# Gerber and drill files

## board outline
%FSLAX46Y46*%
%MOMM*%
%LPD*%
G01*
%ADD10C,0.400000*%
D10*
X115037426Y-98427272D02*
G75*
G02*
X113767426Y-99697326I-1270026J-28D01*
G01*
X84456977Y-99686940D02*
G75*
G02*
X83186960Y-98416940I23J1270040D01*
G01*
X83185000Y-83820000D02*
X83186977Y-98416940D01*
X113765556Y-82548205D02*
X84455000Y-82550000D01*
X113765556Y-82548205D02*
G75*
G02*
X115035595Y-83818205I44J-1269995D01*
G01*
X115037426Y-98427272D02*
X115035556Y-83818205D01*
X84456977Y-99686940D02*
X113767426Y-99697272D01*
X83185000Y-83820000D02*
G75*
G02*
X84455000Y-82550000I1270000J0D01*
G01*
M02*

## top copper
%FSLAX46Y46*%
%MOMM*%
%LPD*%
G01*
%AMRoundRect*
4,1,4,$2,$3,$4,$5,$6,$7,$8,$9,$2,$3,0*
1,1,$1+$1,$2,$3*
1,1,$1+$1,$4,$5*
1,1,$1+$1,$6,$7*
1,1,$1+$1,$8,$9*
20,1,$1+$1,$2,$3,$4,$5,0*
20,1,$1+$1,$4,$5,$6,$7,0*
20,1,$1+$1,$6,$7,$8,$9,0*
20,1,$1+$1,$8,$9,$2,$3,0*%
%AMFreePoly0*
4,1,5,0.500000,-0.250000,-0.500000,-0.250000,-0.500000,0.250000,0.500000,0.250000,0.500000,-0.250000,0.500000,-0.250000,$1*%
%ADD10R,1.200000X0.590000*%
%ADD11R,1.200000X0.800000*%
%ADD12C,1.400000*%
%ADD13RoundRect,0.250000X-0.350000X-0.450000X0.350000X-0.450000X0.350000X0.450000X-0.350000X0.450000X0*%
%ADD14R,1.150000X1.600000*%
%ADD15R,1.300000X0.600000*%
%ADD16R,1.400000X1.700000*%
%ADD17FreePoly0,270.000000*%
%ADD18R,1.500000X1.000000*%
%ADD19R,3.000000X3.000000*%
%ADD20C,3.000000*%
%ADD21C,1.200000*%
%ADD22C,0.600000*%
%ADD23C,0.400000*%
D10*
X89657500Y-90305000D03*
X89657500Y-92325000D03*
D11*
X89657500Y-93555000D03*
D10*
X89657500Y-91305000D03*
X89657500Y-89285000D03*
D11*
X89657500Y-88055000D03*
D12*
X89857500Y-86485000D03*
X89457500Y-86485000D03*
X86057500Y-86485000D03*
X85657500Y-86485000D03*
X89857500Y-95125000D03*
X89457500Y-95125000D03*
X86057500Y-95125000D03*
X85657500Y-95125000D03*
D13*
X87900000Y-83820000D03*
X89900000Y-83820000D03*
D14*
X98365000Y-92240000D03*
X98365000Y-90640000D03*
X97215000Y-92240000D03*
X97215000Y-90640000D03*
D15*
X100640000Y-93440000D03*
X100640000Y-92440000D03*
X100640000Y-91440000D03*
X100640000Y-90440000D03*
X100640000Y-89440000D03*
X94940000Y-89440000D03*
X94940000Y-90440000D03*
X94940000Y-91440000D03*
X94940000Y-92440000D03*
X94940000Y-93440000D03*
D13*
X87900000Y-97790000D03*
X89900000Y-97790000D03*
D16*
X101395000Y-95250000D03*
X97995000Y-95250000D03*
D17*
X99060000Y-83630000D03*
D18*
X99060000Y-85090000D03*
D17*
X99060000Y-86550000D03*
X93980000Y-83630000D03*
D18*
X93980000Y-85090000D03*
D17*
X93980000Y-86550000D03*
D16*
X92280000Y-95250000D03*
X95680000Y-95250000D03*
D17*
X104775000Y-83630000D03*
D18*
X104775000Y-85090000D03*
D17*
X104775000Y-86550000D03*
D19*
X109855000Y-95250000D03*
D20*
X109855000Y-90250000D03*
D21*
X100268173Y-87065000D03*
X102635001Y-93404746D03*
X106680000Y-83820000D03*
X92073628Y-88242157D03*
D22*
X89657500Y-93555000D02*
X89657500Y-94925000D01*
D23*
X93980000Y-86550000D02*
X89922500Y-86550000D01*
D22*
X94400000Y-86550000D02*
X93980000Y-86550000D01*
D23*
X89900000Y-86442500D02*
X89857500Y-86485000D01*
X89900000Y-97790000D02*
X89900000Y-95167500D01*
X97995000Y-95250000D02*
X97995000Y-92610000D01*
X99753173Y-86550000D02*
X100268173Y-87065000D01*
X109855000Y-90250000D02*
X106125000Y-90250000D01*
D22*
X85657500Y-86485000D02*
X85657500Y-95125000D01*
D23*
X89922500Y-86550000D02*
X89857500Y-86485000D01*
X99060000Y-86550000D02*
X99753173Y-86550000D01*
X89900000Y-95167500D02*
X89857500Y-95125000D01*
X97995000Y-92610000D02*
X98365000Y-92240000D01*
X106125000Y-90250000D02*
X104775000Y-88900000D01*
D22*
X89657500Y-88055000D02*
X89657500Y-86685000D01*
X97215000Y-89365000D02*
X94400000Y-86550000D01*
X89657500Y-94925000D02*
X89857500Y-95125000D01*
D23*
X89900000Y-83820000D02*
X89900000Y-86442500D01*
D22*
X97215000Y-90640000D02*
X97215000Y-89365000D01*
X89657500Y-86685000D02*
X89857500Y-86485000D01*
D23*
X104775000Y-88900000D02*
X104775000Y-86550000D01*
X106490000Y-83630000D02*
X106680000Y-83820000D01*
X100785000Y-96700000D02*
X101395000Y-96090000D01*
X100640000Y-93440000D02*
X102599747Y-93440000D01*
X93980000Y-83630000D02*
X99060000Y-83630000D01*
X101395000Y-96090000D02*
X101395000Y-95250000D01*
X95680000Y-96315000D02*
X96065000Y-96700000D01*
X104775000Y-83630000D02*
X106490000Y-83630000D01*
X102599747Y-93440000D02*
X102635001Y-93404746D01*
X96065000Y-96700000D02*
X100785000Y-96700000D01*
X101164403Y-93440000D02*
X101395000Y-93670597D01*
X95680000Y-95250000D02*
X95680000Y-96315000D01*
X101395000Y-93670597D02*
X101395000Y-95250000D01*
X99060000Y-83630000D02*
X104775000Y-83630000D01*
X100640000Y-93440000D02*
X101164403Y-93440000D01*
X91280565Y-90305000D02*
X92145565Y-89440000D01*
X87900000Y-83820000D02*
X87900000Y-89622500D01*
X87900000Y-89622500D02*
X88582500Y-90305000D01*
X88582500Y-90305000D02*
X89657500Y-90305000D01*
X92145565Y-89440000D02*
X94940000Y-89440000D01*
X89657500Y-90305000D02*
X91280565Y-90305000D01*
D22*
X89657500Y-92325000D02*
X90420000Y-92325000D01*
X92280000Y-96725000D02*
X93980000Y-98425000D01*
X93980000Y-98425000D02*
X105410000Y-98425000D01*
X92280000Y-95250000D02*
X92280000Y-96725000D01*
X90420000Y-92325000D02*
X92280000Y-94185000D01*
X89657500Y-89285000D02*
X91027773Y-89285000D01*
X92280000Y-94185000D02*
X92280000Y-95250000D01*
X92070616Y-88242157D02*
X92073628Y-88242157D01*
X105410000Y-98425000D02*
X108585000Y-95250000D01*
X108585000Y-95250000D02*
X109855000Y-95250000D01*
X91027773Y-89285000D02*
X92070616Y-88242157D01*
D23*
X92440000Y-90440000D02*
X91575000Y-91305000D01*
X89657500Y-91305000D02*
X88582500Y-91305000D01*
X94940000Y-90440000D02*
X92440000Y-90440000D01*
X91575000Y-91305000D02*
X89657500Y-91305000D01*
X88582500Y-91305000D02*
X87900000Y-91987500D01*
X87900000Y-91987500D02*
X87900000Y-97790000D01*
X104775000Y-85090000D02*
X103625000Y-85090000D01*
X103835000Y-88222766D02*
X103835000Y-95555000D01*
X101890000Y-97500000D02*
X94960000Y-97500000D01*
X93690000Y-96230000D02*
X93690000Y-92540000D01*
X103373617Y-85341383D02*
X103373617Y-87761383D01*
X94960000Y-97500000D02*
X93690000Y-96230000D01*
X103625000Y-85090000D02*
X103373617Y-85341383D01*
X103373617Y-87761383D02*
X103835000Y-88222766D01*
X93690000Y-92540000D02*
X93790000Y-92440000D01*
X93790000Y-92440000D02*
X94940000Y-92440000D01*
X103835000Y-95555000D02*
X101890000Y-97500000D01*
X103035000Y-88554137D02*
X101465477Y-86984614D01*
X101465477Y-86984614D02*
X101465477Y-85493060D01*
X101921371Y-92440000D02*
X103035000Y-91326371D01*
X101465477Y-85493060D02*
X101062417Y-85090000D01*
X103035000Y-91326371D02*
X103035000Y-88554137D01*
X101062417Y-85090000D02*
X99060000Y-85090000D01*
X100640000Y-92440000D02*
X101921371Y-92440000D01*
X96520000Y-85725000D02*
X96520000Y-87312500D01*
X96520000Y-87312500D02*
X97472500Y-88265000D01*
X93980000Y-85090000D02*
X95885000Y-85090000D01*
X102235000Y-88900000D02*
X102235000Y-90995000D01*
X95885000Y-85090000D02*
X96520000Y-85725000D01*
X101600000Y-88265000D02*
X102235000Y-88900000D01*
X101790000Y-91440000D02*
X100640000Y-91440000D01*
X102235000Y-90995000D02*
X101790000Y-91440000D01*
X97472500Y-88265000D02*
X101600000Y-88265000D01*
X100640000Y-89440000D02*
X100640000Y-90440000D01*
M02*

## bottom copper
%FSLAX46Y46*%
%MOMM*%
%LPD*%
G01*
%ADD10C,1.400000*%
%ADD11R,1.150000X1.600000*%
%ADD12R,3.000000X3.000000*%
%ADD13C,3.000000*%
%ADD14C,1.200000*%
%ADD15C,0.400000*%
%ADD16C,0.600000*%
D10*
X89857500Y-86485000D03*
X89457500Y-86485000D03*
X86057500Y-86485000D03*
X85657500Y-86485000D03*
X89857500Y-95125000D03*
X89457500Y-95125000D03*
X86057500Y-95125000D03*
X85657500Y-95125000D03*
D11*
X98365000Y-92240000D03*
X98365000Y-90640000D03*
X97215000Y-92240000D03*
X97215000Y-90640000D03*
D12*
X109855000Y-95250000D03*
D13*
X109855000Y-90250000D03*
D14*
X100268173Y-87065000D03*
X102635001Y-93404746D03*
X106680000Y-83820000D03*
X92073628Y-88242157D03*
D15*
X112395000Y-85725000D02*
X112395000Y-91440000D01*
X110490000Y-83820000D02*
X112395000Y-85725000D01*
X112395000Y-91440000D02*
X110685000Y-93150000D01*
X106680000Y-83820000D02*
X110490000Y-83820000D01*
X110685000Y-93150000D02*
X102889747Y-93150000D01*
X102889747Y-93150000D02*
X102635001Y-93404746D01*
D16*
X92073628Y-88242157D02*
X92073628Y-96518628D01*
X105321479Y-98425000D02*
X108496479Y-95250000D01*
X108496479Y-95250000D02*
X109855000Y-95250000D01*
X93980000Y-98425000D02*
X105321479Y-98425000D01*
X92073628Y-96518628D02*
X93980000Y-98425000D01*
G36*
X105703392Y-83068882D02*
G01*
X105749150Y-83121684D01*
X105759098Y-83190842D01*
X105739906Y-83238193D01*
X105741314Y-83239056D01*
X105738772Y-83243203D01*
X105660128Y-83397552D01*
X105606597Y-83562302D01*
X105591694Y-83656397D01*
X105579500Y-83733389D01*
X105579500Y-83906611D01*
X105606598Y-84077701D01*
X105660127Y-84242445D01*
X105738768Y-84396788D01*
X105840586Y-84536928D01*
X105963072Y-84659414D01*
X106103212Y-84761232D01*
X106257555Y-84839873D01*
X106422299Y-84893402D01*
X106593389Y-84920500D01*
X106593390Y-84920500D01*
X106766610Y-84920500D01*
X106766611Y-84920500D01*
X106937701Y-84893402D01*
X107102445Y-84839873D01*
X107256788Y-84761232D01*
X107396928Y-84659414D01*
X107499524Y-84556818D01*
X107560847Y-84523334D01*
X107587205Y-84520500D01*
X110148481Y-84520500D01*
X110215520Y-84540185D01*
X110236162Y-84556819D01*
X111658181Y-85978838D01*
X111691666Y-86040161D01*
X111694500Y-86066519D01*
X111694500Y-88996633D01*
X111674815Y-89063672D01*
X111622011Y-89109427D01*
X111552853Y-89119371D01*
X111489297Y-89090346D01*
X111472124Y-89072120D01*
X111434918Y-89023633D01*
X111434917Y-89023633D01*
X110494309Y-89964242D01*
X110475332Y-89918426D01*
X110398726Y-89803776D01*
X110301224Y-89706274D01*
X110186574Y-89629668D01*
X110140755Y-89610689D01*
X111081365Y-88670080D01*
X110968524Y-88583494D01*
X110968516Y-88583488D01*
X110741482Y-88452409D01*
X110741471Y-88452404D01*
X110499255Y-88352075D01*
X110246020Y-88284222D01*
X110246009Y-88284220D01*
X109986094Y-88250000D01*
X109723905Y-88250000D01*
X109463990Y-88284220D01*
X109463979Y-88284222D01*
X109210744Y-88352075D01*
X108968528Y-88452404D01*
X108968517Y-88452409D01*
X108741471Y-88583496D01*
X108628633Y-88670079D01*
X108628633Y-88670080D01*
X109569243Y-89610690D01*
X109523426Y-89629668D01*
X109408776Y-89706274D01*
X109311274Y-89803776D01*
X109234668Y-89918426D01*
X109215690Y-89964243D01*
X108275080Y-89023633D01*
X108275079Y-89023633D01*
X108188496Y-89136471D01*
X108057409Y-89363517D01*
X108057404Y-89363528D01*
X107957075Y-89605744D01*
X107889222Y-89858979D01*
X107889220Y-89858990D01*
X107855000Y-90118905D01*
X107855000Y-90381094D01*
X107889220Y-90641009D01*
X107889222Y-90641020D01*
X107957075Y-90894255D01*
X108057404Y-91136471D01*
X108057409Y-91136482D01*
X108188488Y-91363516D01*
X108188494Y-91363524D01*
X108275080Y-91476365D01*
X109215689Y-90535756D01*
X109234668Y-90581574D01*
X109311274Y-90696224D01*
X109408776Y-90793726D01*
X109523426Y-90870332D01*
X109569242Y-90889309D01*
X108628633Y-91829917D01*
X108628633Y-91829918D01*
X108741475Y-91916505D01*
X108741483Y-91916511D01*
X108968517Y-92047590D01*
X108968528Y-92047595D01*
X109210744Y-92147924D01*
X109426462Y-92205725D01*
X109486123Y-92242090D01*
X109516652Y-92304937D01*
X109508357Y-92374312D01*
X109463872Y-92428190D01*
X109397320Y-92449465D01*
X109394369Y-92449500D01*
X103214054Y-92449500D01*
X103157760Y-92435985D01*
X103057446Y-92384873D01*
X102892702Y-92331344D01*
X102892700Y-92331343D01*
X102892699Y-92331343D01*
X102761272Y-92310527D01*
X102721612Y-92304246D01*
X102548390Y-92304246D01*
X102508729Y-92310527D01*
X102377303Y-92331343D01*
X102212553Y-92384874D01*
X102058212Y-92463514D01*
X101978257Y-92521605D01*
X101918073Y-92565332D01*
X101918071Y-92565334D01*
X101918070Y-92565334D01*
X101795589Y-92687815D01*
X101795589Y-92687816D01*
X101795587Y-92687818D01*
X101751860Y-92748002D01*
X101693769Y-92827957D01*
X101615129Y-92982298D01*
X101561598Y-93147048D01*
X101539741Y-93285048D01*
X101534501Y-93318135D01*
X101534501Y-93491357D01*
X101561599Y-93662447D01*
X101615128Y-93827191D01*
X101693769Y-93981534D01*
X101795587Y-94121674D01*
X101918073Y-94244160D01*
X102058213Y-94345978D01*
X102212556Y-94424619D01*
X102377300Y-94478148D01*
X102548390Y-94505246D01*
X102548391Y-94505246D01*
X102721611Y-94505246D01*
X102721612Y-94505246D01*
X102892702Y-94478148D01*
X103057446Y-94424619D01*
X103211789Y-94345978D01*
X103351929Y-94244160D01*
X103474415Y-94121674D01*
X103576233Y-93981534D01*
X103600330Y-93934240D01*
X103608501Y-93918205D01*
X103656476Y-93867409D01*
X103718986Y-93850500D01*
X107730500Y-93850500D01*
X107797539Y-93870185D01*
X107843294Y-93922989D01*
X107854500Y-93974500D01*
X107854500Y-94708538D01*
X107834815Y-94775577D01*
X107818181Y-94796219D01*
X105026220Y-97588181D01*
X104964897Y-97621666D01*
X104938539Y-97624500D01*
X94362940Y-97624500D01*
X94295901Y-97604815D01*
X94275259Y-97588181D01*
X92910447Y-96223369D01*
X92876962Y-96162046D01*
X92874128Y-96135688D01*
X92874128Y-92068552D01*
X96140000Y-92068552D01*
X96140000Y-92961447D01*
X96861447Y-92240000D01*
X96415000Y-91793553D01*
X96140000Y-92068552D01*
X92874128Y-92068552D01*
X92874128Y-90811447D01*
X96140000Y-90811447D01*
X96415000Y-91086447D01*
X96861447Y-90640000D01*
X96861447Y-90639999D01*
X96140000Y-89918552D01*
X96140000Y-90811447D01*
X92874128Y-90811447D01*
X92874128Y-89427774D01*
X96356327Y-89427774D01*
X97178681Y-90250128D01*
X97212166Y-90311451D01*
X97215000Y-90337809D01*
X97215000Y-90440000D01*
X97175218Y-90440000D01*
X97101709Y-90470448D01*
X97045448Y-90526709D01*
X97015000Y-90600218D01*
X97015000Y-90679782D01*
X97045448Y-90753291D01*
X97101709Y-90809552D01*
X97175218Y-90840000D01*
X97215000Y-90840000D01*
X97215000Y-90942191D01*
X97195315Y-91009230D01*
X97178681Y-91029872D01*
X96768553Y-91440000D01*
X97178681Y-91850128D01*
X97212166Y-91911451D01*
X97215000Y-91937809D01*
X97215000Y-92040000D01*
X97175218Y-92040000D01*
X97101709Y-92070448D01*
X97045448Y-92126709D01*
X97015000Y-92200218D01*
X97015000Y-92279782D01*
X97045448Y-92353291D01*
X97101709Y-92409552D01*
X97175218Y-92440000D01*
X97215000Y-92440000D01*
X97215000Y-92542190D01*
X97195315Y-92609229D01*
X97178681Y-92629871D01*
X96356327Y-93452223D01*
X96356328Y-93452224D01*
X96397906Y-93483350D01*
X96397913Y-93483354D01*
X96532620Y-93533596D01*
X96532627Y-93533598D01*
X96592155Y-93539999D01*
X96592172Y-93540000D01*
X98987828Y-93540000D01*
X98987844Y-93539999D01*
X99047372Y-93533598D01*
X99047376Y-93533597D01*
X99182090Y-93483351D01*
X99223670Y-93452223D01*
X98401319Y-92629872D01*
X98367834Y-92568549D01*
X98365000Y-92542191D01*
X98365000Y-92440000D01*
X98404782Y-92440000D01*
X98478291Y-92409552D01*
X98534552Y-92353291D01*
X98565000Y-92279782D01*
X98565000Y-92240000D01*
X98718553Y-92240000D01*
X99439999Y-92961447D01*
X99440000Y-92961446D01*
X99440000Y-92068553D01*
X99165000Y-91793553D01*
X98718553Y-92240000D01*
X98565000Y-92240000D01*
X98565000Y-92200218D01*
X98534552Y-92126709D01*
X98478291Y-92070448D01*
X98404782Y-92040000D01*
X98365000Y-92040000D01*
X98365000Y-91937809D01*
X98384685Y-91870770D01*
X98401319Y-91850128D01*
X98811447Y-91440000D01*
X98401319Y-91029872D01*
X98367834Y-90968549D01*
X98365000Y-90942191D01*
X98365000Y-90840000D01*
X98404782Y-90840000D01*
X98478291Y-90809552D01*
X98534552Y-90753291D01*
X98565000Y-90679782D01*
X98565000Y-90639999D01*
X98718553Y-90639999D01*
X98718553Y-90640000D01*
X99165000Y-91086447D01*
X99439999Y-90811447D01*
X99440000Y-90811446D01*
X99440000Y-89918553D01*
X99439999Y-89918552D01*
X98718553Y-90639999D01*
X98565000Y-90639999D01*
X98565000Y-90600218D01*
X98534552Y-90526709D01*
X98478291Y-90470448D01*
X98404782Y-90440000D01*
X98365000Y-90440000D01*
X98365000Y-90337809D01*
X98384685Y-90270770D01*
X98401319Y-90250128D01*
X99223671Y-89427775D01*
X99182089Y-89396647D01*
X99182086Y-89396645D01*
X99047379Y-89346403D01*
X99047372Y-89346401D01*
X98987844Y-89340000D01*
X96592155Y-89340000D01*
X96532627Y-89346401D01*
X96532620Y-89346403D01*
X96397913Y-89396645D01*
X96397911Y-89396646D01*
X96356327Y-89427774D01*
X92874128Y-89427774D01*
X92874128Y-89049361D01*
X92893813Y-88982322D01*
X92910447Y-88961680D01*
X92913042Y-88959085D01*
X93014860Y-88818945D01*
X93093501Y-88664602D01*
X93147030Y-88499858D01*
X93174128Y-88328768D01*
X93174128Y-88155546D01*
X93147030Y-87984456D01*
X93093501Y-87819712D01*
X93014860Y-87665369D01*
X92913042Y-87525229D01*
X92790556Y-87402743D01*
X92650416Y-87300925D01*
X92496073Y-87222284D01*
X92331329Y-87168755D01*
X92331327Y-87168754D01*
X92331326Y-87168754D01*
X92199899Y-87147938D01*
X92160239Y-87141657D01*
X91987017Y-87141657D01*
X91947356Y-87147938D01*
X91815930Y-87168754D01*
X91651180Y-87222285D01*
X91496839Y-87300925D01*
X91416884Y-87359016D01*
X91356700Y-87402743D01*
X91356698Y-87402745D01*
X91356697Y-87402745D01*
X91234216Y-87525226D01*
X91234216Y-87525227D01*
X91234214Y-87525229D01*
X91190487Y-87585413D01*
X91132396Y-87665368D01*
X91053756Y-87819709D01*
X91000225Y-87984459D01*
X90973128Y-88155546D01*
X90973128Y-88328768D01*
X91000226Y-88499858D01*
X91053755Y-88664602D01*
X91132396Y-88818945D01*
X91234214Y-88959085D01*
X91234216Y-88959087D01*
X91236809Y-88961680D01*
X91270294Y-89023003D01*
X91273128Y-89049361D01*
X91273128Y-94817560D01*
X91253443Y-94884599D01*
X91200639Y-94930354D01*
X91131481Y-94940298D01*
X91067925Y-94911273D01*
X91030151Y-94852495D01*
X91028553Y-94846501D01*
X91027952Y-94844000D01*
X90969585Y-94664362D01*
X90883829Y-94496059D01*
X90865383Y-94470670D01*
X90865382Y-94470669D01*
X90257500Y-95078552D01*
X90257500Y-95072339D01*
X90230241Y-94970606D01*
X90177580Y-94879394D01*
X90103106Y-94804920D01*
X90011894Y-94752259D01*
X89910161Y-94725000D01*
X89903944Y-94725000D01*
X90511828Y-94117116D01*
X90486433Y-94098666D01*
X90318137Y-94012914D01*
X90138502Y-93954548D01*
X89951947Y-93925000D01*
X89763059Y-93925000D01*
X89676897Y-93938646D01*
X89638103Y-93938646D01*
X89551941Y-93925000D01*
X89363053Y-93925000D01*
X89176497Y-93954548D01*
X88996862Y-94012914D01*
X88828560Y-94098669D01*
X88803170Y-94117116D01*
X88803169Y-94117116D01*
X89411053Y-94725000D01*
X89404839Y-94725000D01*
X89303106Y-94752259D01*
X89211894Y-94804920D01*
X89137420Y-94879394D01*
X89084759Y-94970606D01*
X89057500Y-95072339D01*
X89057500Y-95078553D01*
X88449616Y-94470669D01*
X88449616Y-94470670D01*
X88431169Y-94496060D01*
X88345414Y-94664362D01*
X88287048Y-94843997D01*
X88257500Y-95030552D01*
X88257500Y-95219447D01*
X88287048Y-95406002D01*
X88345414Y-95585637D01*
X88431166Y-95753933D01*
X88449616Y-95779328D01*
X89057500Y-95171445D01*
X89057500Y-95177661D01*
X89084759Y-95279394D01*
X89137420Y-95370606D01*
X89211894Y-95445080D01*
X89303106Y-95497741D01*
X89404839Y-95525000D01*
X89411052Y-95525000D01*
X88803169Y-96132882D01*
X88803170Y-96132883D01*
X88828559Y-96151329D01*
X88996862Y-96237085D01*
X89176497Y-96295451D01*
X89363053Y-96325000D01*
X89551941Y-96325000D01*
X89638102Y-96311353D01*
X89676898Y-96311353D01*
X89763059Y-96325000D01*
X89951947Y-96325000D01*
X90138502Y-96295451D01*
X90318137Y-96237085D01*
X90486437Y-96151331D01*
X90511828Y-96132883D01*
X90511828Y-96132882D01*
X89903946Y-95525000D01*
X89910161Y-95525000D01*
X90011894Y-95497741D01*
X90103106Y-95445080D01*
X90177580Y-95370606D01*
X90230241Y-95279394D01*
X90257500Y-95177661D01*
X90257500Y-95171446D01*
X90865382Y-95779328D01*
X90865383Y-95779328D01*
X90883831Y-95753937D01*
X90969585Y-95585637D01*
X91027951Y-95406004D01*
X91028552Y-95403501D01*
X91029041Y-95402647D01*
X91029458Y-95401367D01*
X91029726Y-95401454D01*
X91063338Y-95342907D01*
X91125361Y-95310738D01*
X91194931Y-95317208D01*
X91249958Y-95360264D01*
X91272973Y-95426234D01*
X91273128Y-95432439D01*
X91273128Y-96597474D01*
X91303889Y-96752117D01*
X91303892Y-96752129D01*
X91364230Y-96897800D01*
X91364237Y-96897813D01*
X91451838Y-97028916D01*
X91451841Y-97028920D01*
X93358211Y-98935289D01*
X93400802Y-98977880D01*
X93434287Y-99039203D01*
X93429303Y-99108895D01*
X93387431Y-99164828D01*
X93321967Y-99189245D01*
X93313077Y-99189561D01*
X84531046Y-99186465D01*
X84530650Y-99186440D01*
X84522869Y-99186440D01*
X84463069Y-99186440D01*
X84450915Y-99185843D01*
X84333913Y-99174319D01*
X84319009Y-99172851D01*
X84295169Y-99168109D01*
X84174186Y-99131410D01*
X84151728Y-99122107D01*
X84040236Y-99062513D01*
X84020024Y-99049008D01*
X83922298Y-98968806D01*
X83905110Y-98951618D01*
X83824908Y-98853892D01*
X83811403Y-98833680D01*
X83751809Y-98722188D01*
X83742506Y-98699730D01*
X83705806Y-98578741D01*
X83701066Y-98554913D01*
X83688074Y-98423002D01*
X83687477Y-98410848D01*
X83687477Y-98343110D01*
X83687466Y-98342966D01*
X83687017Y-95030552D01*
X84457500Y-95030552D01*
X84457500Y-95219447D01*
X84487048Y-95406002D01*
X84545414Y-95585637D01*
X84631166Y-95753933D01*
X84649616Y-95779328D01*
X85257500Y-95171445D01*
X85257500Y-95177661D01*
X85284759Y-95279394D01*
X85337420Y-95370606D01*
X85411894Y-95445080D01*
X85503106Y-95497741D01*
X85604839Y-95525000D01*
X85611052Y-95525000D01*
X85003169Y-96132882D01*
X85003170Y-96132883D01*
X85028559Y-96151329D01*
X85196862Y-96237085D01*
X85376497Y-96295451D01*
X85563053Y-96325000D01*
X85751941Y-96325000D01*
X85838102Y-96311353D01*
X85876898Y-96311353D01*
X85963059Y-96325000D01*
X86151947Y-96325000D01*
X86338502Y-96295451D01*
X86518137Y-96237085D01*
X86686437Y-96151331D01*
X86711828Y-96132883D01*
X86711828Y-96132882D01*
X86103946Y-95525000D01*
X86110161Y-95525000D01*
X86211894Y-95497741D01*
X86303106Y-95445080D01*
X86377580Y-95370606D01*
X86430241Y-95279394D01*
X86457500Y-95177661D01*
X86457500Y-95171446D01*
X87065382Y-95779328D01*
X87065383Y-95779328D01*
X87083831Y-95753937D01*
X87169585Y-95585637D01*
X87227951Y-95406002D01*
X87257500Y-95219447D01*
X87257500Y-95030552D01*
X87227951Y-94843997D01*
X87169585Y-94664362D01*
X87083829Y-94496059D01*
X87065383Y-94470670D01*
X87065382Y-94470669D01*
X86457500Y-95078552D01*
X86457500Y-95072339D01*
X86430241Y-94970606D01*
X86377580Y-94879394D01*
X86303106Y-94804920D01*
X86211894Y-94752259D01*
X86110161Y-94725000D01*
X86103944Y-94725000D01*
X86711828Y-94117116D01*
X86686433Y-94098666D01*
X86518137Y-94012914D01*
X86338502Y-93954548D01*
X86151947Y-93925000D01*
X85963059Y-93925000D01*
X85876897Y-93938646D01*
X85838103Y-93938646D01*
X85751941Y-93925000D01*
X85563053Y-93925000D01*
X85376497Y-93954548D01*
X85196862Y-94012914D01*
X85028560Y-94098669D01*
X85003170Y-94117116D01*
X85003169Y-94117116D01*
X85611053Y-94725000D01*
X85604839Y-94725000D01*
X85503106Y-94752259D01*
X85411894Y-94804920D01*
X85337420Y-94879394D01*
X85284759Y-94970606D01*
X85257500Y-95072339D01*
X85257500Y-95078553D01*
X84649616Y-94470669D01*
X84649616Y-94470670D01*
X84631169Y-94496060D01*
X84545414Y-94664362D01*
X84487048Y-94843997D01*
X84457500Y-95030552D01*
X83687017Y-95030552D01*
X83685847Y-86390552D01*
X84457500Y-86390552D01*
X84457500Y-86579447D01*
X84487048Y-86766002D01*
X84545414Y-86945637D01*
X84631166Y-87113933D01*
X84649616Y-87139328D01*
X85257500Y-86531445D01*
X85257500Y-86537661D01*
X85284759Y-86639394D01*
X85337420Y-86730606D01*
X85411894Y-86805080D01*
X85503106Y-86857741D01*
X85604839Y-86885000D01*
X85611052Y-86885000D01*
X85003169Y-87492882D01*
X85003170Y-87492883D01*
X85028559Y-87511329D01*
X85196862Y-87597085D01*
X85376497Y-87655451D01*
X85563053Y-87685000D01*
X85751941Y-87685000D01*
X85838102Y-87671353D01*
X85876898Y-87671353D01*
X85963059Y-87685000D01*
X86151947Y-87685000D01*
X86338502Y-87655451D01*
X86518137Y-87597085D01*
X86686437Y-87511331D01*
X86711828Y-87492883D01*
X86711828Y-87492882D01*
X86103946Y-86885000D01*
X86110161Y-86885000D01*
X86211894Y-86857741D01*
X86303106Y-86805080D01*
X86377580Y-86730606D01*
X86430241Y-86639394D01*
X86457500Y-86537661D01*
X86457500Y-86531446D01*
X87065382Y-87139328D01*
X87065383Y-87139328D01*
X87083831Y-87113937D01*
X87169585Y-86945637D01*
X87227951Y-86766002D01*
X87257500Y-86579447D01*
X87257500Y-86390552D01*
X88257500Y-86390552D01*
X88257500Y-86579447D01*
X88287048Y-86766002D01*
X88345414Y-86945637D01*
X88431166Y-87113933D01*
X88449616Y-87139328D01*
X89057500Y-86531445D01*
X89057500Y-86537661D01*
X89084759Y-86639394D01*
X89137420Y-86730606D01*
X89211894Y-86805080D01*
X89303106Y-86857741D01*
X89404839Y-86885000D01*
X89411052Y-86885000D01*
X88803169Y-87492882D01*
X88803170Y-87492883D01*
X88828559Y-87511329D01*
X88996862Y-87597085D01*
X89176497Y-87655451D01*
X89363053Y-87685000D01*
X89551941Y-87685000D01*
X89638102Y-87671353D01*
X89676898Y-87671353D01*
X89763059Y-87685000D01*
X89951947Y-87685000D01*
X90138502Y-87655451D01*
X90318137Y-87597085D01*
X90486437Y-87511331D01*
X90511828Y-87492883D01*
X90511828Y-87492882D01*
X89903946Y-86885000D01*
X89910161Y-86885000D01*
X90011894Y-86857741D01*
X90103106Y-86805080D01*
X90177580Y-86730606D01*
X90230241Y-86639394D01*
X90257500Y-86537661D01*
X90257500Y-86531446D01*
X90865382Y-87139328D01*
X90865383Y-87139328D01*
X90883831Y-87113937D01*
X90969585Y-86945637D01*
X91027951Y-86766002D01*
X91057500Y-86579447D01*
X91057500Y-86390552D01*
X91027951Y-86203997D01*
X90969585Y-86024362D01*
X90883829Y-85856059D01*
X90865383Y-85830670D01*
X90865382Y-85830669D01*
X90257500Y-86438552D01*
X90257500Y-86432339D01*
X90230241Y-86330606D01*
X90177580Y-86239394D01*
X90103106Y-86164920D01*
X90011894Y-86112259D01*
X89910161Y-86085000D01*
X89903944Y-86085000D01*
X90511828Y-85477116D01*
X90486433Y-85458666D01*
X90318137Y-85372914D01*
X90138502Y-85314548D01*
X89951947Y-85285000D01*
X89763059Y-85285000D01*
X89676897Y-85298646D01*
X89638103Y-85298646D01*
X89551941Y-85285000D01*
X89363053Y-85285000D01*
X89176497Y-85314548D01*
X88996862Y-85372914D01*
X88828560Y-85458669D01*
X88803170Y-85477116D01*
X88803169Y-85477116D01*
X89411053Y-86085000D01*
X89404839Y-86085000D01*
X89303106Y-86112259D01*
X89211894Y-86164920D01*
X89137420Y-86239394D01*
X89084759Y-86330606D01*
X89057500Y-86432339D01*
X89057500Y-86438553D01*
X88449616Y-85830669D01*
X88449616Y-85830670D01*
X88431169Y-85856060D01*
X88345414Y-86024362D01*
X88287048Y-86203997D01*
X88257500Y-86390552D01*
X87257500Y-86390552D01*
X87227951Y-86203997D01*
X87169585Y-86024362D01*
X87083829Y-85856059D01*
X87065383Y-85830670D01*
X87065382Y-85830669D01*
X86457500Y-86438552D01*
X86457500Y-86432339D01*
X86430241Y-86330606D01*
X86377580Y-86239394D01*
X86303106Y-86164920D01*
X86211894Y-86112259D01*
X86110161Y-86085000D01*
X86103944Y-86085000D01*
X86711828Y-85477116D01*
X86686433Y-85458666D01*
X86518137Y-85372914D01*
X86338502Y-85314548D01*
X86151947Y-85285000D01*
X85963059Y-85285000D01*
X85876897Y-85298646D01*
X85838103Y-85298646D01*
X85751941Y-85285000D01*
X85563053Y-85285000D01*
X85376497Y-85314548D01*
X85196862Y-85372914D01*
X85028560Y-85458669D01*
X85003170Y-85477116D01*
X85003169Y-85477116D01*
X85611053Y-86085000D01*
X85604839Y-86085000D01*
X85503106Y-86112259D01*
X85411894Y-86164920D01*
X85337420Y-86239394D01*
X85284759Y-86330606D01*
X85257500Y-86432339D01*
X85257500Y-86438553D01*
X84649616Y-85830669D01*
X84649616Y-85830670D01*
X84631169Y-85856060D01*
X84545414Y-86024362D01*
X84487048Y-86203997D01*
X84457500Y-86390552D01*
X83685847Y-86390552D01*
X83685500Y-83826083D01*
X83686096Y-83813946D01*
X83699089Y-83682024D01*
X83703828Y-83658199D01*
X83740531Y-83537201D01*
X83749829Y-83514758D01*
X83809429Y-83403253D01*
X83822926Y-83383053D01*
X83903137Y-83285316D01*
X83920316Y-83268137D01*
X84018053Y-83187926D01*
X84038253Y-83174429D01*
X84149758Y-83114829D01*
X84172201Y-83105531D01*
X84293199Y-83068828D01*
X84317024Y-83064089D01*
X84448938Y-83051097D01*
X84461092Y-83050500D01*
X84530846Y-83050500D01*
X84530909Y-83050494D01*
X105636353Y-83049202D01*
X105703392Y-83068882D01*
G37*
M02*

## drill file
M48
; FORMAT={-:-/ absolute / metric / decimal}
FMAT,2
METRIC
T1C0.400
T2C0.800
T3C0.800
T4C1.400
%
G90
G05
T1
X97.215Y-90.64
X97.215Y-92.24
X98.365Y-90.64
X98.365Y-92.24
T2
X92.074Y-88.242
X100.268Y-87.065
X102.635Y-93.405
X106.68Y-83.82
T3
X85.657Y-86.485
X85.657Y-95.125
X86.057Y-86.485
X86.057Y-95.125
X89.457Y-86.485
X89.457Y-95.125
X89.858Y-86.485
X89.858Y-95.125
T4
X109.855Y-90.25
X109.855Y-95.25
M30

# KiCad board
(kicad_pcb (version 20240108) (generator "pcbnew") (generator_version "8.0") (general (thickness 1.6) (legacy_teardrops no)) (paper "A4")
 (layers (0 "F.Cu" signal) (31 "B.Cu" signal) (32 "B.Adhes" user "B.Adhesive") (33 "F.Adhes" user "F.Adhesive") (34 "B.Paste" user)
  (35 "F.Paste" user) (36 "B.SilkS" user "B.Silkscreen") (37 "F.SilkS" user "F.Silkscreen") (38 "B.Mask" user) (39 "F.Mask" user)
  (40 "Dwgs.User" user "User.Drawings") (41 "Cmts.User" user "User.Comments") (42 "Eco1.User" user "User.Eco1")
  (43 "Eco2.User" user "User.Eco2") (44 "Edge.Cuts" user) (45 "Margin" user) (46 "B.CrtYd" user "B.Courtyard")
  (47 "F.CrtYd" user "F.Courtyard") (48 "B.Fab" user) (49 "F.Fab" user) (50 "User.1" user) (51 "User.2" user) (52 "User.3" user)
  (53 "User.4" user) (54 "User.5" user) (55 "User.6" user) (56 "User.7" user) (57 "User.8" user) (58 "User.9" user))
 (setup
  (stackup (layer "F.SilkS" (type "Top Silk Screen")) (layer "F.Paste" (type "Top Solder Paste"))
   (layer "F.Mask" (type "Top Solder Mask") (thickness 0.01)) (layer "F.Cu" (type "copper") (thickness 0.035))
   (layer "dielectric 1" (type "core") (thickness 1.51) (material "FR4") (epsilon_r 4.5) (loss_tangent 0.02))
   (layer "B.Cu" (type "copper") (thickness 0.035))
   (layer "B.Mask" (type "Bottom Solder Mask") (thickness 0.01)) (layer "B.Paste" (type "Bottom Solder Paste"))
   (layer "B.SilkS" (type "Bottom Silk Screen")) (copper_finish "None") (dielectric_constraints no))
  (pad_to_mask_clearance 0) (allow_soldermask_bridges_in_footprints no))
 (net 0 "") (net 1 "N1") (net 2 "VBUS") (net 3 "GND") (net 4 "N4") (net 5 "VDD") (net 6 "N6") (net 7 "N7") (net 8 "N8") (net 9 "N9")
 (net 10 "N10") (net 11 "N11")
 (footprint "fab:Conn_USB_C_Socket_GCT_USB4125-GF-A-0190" (layer "F.Cu") (at 89.6575 90.805 -90)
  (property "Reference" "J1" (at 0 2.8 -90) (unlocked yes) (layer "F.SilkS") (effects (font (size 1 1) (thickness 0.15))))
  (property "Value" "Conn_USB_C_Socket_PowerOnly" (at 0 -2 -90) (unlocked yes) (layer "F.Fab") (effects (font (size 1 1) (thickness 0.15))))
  (pad "A5" smd rect (at -0.5 0 270) (size 0.59 1.2) (layers "F.Cu" "F.Paste" "F.Mask") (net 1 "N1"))
  (pad "A9" smd rect (at 1.52 0 270) (size 0.59 1.2) (layers "F.Cu" "F.Paste" "F.Mask") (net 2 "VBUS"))
  (pad "A12" smd rect (at 2.75 0 270) (size 0.8 1.2) (layers "F.Cu" "F.Paste" "F.Mask") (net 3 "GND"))
  (pad "B5" smd rect (at 0.5 0 270) (size 0.59 1.2) (layers "F.Cu" "F.Paste" "F.Mask") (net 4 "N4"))
  (pad "B9" smd rect (at -1.52 0 270) (size 0.59 1.2) (layers "F.Cu" "F.Paste" "F.Mask") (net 2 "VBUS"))
  (pad "B12" smd rect (at -2.75 0 270) (size 0.8 1.2) (layers "F.Cu" "F.Paste" "F.Mask") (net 3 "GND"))
  (pad "S1" thru_hole circle (at -4.32 -0.2 270) (size 1.4 1.4) (drill 0.8) (layers "*.Cu" "*.Mask") (remove_unused_layers no) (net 3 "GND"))
  (pad "S1" thru_hole circle (at -4.32 0.2 270) (size 1.4 1.4) (drill 0.8) (layers "*.Cu" "*.Mask") (remove_unused_layers no) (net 3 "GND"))
  (pad "S1" thru_hole circle (at -4.32 3.6 270) (size 1.4 1.4) (drill 0.8) (layers "*.Cu" "*.Mask") (remove_unused_layers no) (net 3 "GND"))
  (pad "S1" thru_hole circle (at -4.32 4 270) (size 1.4 1.4) (drill 0.8) (layers "*.Cu" "*.Mask") (remove_unused_layers no) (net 3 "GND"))
  (pad "S1" thru_hole circle (at 4.32 -0.2 270) (size 1.4 1.4) (drill 0.8) (layers "*.Cu" "*.Mask") (remove_unused_layers no) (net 3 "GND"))
  (pad "S1" thru_hole circle (at 4.32 0.2 270) (size 1.4 1.4) (drill 0.8) (layers "*.Cu" "*.Mask") (remove_unused_layers no) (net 3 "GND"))
  (pad "S1" thru_hole circle (at 4.32 3.6 270) (size 1.4 1.4) (drill 0.8) (layers "*.Cu" "*.Mask") (remove_unused_layers no) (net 3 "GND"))
  (pad "S1" thru_hole circle (at 4.32 4 270) (size 1.4 1.4) (drill 0.8) (layers "*.Cu" "*.Mask") (remove_unused_layers no) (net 3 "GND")))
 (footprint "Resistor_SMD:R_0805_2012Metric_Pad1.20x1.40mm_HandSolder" (layer "F.Cu") (at 88.9 83.82)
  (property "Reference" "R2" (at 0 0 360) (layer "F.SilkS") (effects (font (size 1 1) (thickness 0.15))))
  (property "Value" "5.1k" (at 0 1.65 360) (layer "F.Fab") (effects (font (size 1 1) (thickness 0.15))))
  (pad "1" smd roundrect (at -1 0) (size 1.2 1.4) (layers "F.Cu" "F.Paste" "F.Mask") (roundrect_rratio 0.208333) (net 1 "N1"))
  (pad "2" smd roundrect (at 1 0) (size 1.2 1.4) (layers "F.Cu" "F.Paste" "F.Mask") (roundrect_rratio 0.208333) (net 3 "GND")))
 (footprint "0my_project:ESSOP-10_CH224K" (layer "F.Cu") (at 97.79 91.44 180)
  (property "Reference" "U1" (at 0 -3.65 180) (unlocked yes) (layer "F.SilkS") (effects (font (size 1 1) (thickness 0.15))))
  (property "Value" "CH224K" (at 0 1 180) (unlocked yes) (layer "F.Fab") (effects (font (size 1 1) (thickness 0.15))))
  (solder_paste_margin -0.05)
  (pad "0" thru_hole rect (at -0.575 -0.8 180) (size 1.15 1.6) (drill 0.4) (layers "*.Cu" "*.Mask" "F.Paste") (remove_unused_layers no)
   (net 3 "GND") (solder_paste_margin -0.1) (thermal_bridge_angle 45))
  (pad "0" thru_hole rect (at -0.575 0.8 180) (size 1.15 1.6) (drill 0.4) (layers "*.Cu" "*.Mask" "F.Paste") (remove_unused_layers no)
   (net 3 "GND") (solder_paste_margin -0.1) (thermal_bridge_angle 45))
  (pad "0" thru_hole rect (at 0.575 -0.8 180) (size 1.15 1.6) (drill 0.4) (layers "*.Cu" "*.Mask" "F.Paste") (remove_unused_layers no)
   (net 3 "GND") (solder_paste_margin -0.1) (thermal_bridge_angle 45))
  (pad "0" thru_hole rect (at 0.575 0.8 180) (size 1.15 1.6) (drill 0.4) (layers "*.Cu" "*.Mask" "F.Paste") (remove_unused_layers no)
   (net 3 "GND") (solder_paste_margin -0.1) (thermal_bridge_angle 45))
  (pad "1" smd rect (at -2.85 -2 180) (size 1.3 0.6) (layers "F.Cu" "F.Paste" "F.Mask") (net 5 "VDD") (thermal_bridge_angle 45))
  (pad "2" smd rect (at -2.85 -1 180) (size 1.3 0.6) (layers "F.Cu" "F.Paste" "F.Mask") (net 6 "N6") (thermal_bridge_angle 45))
  (pad "3" smd rect (at -2.85 0 180) (size 1.3 0.6) (layers "F.Cu" "F.Paste" "F.Mask") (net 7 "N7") (thermal_bridge_angle 45))
  (pad "4" smd rect (at -2.85 1 180) (size 1.3 0.6) (layers "F.Cu" "F.Paste" "F.Mask") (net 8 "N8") (thermal_bridge_angle 45))
  (pad "5" smd rect (at -2.85 2 180) (size 1.3 0.6) (layers "F.Cu" "F.Paste" "F.Mask") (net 8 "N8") (thermal_bridge_angle 45))
  (pad "6" smd rect (at 2.85 2 180) (size 1.3 0.6) (layers "F.Cu" "F.Paste" "F.Mask") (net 1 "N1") (thermal_bridge_angle 45))
  (pad "7" smd rect (at 2.85 1 180) (size 1.3 0.6) (layers "F.Cu" "F.Paste" "F.Mask") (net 4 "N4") (thermal_bridge_angle 45))
  (pad "8" smd rect (at 2.85 0 180) (size 1.3 0.6) (layers "F.Cu" "F.Paste" "F.Mask") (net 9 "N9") (thermal_bridge_angle 45))
  (pad "9" smd rect (at 2.85 -1 180) (size 1.3 0.6) (layers "F.Cu" "F.Paste" "F.Mask") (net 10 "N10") (thermal_bridge_angle 45))
  (pad "10" smd rect (at 2.85 -2 180) (size 1.3 0.6) (layers "F.Cu" "F.Paste" "F.Mask") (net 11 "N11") (thermal_bridge_angle 45)))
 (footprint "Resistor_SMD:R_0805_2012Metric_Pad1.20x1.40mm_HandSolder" (layer "F.Cu") (at 88.9 97.79)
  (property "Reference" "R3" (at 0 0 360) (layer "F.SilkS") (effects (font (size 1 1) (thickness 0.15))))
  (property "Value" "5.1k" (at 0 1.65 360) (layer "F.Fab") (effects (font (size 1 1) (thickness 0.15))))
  (pad "1" smd roundrect (at -1 0) (size 1.2 1.4) (layers "F.Cu" "F.Paste" "F.Mask") (roundrect_rratio 0.208333) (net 4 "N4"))
  (pad "2" smd roundrect (at 1 0) (size 1.2 1.4) (layers "F.Cu" "F.Paste" "F.Mask") (roundrect_rratio 0.208333) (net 3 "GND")))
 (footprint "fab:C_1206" (layer "F.Cu") (at 99.695 95.25 180)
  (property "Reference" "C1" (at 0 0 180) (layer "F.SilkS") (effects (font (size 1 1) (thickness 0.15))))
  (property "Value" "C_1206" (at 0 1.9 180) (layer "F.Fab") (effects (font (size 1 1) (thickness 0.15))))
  (pad "1" smd rect (at -1.7 0 180) (size 1.4 1.7) (layers "F.Cu" "F.Paste" "F.Mask") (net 5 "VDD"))
  (pad "2" smd rect (at 1.7 0 180) (size 1.4 1.7) (layers "F.Cu" "F.Paste" "F.Mask") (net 3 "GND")))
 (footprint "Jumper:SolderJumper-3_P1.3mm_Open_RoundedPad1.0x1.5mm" (layer "F.Cu") (at 99.06 85.09 -90)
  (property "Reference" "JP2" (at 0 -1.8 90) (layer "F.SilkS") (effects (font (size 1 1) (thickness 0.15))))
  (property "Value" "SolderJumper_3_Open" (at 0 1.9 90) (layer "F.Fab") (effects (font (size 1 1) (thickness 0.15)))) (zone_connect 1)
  (pad "1" smd custom (at -1.46 0 270) (size 1 0.5) (layers "F.Cu" "F.Mask") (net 5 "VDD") (zone_connect 2) (thermal_bridge_angle 45)
   (options (clearance outline) (anchor rect)) (primitives))
  (pad "2" smd rect (at 0 0 270) (size 1 1.5) (layers "F.Cu" "F.Mask") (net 6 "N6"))
  (pad "3" smd custom (at 1.46 0 270) (size 1 0.5) (layers "F.Cu" "F.Mask") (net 3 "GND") (zone_connect 2) (thermal_bridge_angle 45)
   (options (clearance outline) (anchor rect)) (primitives)))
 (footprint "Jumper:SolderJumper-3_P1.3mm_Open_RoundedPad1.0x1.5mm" (layer "F.Cu") (at 93.98 85.09 -90)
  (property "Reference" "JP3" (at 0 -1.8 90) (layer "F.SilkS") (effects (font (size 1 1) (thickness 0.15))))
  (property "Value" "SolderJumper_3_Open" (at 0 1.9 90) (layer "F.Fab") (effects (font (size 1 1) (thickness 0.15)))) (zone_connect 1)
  (pad "1" smd custom (at -1.46 0 270) (size 1 0.5) (layers "F.Cu" "F.Mask") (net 5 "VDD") (zone_connect 2) (thermal_bridge_angle 45)
   (options (clearance outline) (anchor rect)) (primitives))
  (pad "2" smd rect (at 0 0 270) (size 1 1.5) (layers "F.Cu" "F.Mask") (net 7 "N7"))
  (pad "3" smd custom (at 1.46 0 270) (size 1 0.5) (layers "F.Cu" "F.Mask") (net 3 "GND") (zone_connect 2) (thermal_bridge_angle 45)
   (options (clearance outline) (anchor rect)) (primitives)))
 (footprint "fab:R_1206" (layer "F.Cu") (at 93.98 95.25)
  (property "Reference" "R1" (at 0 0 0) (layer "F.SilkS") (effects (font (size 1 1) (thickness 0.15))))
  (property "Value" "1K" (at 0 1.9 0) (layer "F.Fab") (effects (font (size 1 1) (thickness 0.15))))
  (pad "1" smd rect (at -1.7 0) (size 1.4 1.7) (layers "F.Cu" "F.Paste" "F.Mask") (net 2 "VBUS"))
  (pad "2" smd rect (at 1.7 0) (size 1.4 1.7) (layers "F.Cu" "F.Paste" "F.Mask") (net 5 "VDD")))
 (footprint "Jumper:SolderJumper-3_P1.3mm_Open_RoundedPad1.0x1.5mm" (layer "F.Cu") (at 104.775 85.09 -90)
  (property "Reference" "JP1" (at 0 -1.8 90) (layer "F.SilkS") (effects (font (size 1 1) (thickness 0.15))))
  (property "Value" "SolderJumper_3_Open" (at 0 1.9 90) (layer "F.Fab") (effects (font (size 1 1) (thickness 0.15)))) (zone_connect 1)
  (pad "1" smd custom (at -1.46 0 270) (size 1 0.5) (layers "F.Cu" "F.Mask") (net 5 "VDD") (zone_connect 2) (thermal_bridge_angle 45)
   (options (clearance outline) (anchor rect)) (primitives))
  (pad "2" smd rect (at 0 0 270) (size 1 1.5) (layers "F.Cu" "F.Mask") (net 10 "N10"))
  (pad "3" smd custom (at 1.46 0 270) (size 1 0.5) (layers "F.Cu" "F.Mask") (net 3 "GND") (zone_connect 2) (thermal_bridge_angle 45)
   (options (clearance outline) (anchor rect)) (primitives)))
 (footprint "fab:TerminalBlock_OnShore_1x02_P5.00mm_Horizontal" (layer "F.Cu") (at 109.855 95.25 90)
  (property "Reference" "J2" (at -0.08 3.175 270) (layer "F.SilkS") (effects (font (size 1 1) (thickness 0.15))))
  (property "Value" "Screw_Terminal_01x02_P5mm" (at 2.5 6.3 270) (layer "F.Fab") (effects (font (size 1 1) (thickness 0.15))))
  (pad "1" thru_hole rect (at 0 0 90) (size 3 3) (drill 1.4) (layers "*.Cu" "*.Mask") (remove_unused_layers no) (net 2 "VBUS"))
  (pad "2" thru_hole circle (at 5 0 90) (size 3 3) (drill 1.4) (layers "*.Cu" "*.Mask") (remove_unused_layers no) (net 3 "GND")))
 (gr_arc (start 115.037426 98.427272) (mid 114.665452 99.325298) (end 113.767426 99.697272) (stroke (width 0.4) (type default))
  (layer "Edge.Cuts"))
 (gr_arc (start 84.456977 99.68694) (mid 83.558951 99.314966) (end 83.186977 98.41694) (stroke (width 0.4) (type default))
  (layer "Edge.Cuts"))
 (gr_line (start 83.185 83.82) (end 83.186977 98.41694) (stroke (width 0.4) (type default)) (layer "Edge.Cuts"))
 (gr_line (start 113.765556 82.548205) (end 84.455 82.55) (stroke (width 0.4) (type default)) (layer "Edge.Cuts"))
 (gr_arc (start 113.765556 82.548205) (mid 114.663582 82.920179) (end 115.035556 83.818205) (stroke (width 0.4) (type default))
  (layer "Edge.Cuts"))
 (gr_line (start 115.037426 98.427272) (end 115.035556 83.818205) (stroke (width 0.4) (type default)) (layer "Edge.Cuts"))
 (gr_line (start 84.456977 99.68694) (end 113.767426 99.697272) (stroke (width 0.4) (type default)) (layer "Edge.Cuts"))
 (gr_arc (start 83.185 83.82) (mid 83.556974 82.921974) (end 84.455 82.55) (stroke (width 0.4) (type default)) (layer "Edge.Cuts"))
 (segment (start 89.6575 93.555) (end 89.6575 94.925) (width 0.6) (layer "F.Cu") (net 3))
 (segment (start 93.98 86.55) (end 89.9225 86.55) (width 0.4) (layer "F.Cu") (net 3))
 (segment (start 94.4 86.55) (end 93.98 86.55) (width 0.6) (layer "F.Cu") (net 3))
 (segment (start 89.9 86.4425) (end 89.8575 86.485) (width 0.4) (layer "F.Cu") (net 3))
 (segment (start 89.9 97.79) (end 89.9 95.1675) (width 0.4) (layer "F.Cu") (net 3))
 (segment (start 97.995 95.25) (end 97.995 92.61) (width 0.4) (layer "F.Cu") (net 3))
 (segment (start 99.753173 86.55) (end 100.268173 87.065) (width 0.4) (layer "F.Cu") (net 3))
 (segment (start 109.855 90.25) (end 106.125 90.25) (width 0.4) (layer "F.Cu") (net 3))
 (segment (start 85.6575 86.485) (end 85.6575 95.125) (width 0.6) (layer "F.Cu") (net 3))
 (segment (start 89.9225 86.55) (end 89.8575 86.485) (width 0.4) (layer "F.Cu") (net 3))
 (segment (start 99.06 86.55) (end 99.753173 86.55) (width 0.4) (layer "F.Cu") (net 3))
 (segment (start 89.9 95.1675) (end 89.8575 95.125) (width 0.4) (layer "F.Cu") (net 3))
 (segment (start 97.995 92.61) (end 98.365 92.24) (width 0.4) (layer "F.Cu") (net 3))
 (segment (start 106.125 90.25) (end 104.775 88.9) (width 0.4) (layer "F.Cu") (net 3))
 (segment (start 89.6575 88.055) (end 89.6575 86.685) (width 0.6) (layer "F.Cu") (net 3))
 (segment (start 97.215 89.365) (end 94.4 86.55) (width 0.6) (layer "F.Cu") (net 3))
 (segment (start 89.6575 94.925) (end 89.8575 95.125) (width 0.6) (layer "F.Cu") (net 3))
 (segment (start 89.9 83.82) (end 89.9 86.4425) (width 0.4) (layer "F.Cu") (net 3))
 (segment (start 97.215 90.64) (end 97.215 89.365) (width 0.6) (layer "F.Cu") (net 3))
 (segment (start 89.6575 86.685) (end 89.8575 86.485) (width 0.6) (layer "F.Cu") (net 3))
 (segment (start 104.775 88.9) (end 104.775 86.55) (width 0.4) (layer "F.Cu") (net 3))
 (via (at 100.268173 87.065) (size 1.2) (drill 0.8) (layers "F.Cu" "B.Cu") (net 3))
 (segment (start 106.49 83.63) (end 106.68 83.82) (width 0.4) (layer "F.Cu") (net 5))
 (segment (start 100.785 96.7) (end 101.395 96.09) (width 0.4) (layer "F.Cu") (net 5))
 (segment (start 100.64 93.44) (end 102.599747 93.44) (width 0.4) (layer "F.Cu") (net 5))
 (segment (start 93.98 83.63) (end 99.06 83.63) (width 0.4) (layer "F.Cu") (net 5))
 (segment (start 101.395 96.09) (end 101.395 95.25) (width 0.4) (layer "F.Cu") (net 5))
 (segment (start 95.68 96.315) (end 96.065 96.7) (width 0.4) (layer "F.Cu") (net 5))
 (segment (start 104.775 83.63) (end 106.49 83.63) (width 0.4) (layer "F.Cu") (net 5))
 (segment (start 102.599747 93.44) (end 102.635001 93.404746) (width 0.4) (layer "F.Cu") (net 5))
 (segment (start 96.065 96.7) (end 100.785 96.7) (width 0.4) (layer "F.Cu") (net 5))
 (segment (start 101.164403 93.44) (end 101.395 93.670597) (width 0.4) (layer "F.Cu") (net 5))
 (segment (start 95.68 95.25) (end 95.68 96.315) (width 0.4) (layer "F.Cu") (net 5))
 (segment (start 101.395 93.670597) (end 101.395 95.25) (width 0.4) (layer "F.Cu") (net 5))
 (segment (start 99.06 83.63) (end 104.775 83.63) (width 0.4) (layer "F.Cu") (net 5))
 (segment (start 100.64 93.44) (end 101.164403 93.44) (width 0.4) (layer "F.Cu") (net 5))
 (via (at 102.635001 93.404746) (size 1.2) (drill 0.8) (layers "F.Cu" "B.Cu") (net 5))
 (via (at 106.68 83.82) (size 1.2) (drill 0.8) (layers "F.Cu" "B.Cu") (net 5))
 (segment (start 112.395 85.725) (end 112.395 91.44) (width 0.4) (layer "B.Cu") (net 5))
 (segment (start 110.49 83.82) (end 112.395 85.725) (width 0.4) (layer "B.Cu") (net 5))
 (segment (start 112.395 91.44) (end 110.685 93.15) (width 0.4) (layer "B.Cu") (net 5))
 (segment (start 106.68 83.82) (end 110.49 83.82) (width 0.4) (layer "B.Cu") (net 5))
 (segment (start 110.685 93.15) (end 102.889747 93.15) (width 0.4) (layer "B.Cu") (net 5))
 (segment (start 102.889747 93.15) (end 102.635001 93.404746) (width 0.4) (layer "B.Cu") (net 5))
 (segment (start 91.280565 90.305) (end 92.145565 89.44) (width 0.4) (layer "F.Cu") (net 1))
 (segment (start 87.9 83.82) (end 87.9 89.6225) (width 0.4) (layer "F.Cu") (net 1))
 (segment (start 87.9 89.6225) (end 88.5825 90.305) (width 0.4) (layer "F.Cu") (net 1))
 (segment (start 88.5825 90.305) (end 89.6575 90.305) (width 0.4) (layer "F.Cu") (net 1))
 (segment (start 92.145565 89.44) (end 94.94 89.44) (width 0.4) (layer "F.Cu") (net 1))
 (segment (start 89.6575 90.305) (end 91.280565 90.305) (width 0.4) (layer "F.Cu") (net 1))
 (segment (start 89.6575 92.325) (end 90.42 92.325) (width 0.6) (layer "F.Cu") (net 2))
 (segment (start 92.28 96.725) (end 93.98 98.425) (width 0.6) (layer "F.Cu") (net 2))
 (segment (start 93.98 98.425) (end 105.41 98.425) (width 0.6) (layer "F.Cu") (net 2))
 (segment (start 92.28 95.25) (end 92.28 96.725) (width 0.6) (layer "F.Cu") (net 2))
 (segment (start 90.42 92.325) (end 92.28 94.185) (width 0.6) (layer "F.Cu") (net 2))
 (segment (start 89.6575 89.285) (end 91.027773 89.285) (width 0.6) (layer "F.Cu") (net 2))
 (segment (start 92.28 94.185) (end 92.28 95.25) (width 0.6) (layer "F.Cu") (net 2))
 (segment (start 92.070616 88.242157) (end 92.073628 88.242157) (width 0.6) (layer "F.Cu") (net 2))
 (segment (start 105.41 98.425) (end 108.585 95.25) (width 0.6) (layer "F.Cu") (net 2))
 (segment (start 108.585 95.25) (end 109.855 95.25) (width 0.6) (layer "F.Cu") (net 2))
 (segment (start 91.027773 89.285) (end 92.070616 88.242157) (width 0.6) (layer "F.Cu") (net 2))
 (via (at 92.073628 88.242157) (size 1.2) (drill 0.8) (layers "F.Cu" "B.Cu") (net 2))
 (segment (start 92.073628 88.242157) (end 92.073628 96.518628) (width 0.6) (layer "B.Cu") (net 2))
 (segment (start 105.321479 98.425) (end 108.496479 95.25) (width 0.6) (layer "B.Cu") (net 2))
 (segment (start 108.496479 95.25) (end 109.855 95.25) (width 0.6) (layer "B.Cu") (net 2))
 (segment (start 93.98 98.425) (end 105.321479 98.425) (width 0.6) (layer "B.Cu") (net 2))
 (segment (start 92.073628 96.518628) (end 93.98 98.425) (width 0.6) (layer "B.Cu") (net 2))
 (segment (start 92.44 90.44) (end 91.575 91.305) (width 0.4) (layer "F.Cu") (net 4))
 (segment (start 89.6575 91.305) (end 88.5825 91.305) (width 0.4) (layer "F.Cu") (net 4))
 (segment (start 94.94 90.44) (end 92.44 90.44) (width 0.4) (layer "F.Cu") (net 4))
 (segment (start 91.575 91.305) (end 89.6575 91.305) (width 0.4) (layer "F.Cu") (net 4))
 (segment (start 88.5825 91.305) (end 87.9 91.9875) (width 0.4) (layer "F.Cu") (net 4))
 (segment (start 87.9 91.9875) (end 87.9 97.79) (width 0.4) (layer "F.Cu") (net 4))
 (segment (start 104.775 85.09) (end 103.625 85.09) (width 0.4) (layer "F.Cu") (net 10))
 (segment (start 103.835 88.222766) (end 103.835 95.555) (width 0.4) (layer "F.Cu") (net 10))
 (segment (start 101.89 97.5) (end 94.96 97.5) (width 0.4) (layer "F.Cu") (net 10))
 (segment (start 93.69 96.23) (end 93.69 92.54) (width 0.4) (layer "F.Cu") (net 10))
 (segment (start 103.373617 85.341383) (end 103.373617 87.761383) (width 0.4) (layer "F.Cu") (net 10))
 (segment (start 94.96 97.5) (end 93.69 96.23) (width 0.4) (layer "F.Cu") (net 10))
 (segment (start 103.625 85.09) (end 103.373617 85.341383) (width 0.4) (layer "F.Cu") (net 10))
 (segment (start 103.373617 87.761383) (end 103.835 88.222766) (width 0.4) (layer "F.Cu") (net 10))
 (segment (start 93.69 92.54) (end 93.79 92.44) (width 0.4) (layer "F.Cu") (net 10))
 (segment (start 93.79 92.44) (end 94.94 92.44) (width 0.4) (layer "F.Cu") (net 10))
 (segment (start 103.835 95.555) (end 101.89 97.5) (width 0.4) (layer "F.Cu") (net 10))
 (segment (start 103.035 88.554137) (end 101.465477 86.984614) (width 0.4) (layer "F.Cu") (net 6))
 (segment (start 101.465477 86.984614) (end 101.465477 85.49306) (width 0.4) (layer "F.Cu") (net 6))
 (segment (start 101.921371 92.44) (end 103.035 91.326371) (width 0.4) (layer "F.Cu") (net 6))
 (segment (start 101.465477 85.49306) (end 101.062417 85.09) (width 0.4) (layer "F.Cu") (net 6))
 (segment (start 103.035 91.326371) (end 103.035 88.554137) (width 0.4) (layer "F.Cu") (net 6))
 (segment (start 101.062417 85.09) (end 99.06 85.09) (width 0.4) (layer "F.Cu") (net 6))
 (segment (start 100.64 92.44) (end 101.921371 92.44) (width 0.4) (layer "F.Cu") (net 6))
 (segment (start 96.52 85.725) (end 96.52 87.3125) (width 0.4) (layer "F.Cu") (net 7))
 (segment (start 96.52 87.3125) (end 97.4725 88.265) (width 0.4) (layer "F.Cu") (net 7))
 (segment (start 93.98 85.09) (end 95.885 85.09) (width 0.4) (layer "F.Cu") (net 7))
 (segment (start 102.235 88.9) (end 102.235 90.995) (width 0.4) (layer "F.Cu") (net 7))
 (segment (start 95.885 85.09) (end 96.52 85.725) (width 0.4) (layer "F.Cu") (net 7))
 (segment (start 101.6 88.265) (end 102.235 88.9) (width 0.4) (layer "F.Cu") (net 7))
 (segment (start 101.79 91.44) (end 100.64 91.44) (width 0.4) (layer "F.Cu") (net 7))
 (segment (start 102.235 90.995) (end 101.79 91.44) (width 0.4) (layer "F.Cu") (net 7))
 (segment (start 97.4725 88.265) (end 101.6 88.265) (width 0.4) (layer "F.Cu") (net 7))
 (segment (start 100.64 89.44) (end 100.64 90.44) (width 0.4) (layer "F.Cu") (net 8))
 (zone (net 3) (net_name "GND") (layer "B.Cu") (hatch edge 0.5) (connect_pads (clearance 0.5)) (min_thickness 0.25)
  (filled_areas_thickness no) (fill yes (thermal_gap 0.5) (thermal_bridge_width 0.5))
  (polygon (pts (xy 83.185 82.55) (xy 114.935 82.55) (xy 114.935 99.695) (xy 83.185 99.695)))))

